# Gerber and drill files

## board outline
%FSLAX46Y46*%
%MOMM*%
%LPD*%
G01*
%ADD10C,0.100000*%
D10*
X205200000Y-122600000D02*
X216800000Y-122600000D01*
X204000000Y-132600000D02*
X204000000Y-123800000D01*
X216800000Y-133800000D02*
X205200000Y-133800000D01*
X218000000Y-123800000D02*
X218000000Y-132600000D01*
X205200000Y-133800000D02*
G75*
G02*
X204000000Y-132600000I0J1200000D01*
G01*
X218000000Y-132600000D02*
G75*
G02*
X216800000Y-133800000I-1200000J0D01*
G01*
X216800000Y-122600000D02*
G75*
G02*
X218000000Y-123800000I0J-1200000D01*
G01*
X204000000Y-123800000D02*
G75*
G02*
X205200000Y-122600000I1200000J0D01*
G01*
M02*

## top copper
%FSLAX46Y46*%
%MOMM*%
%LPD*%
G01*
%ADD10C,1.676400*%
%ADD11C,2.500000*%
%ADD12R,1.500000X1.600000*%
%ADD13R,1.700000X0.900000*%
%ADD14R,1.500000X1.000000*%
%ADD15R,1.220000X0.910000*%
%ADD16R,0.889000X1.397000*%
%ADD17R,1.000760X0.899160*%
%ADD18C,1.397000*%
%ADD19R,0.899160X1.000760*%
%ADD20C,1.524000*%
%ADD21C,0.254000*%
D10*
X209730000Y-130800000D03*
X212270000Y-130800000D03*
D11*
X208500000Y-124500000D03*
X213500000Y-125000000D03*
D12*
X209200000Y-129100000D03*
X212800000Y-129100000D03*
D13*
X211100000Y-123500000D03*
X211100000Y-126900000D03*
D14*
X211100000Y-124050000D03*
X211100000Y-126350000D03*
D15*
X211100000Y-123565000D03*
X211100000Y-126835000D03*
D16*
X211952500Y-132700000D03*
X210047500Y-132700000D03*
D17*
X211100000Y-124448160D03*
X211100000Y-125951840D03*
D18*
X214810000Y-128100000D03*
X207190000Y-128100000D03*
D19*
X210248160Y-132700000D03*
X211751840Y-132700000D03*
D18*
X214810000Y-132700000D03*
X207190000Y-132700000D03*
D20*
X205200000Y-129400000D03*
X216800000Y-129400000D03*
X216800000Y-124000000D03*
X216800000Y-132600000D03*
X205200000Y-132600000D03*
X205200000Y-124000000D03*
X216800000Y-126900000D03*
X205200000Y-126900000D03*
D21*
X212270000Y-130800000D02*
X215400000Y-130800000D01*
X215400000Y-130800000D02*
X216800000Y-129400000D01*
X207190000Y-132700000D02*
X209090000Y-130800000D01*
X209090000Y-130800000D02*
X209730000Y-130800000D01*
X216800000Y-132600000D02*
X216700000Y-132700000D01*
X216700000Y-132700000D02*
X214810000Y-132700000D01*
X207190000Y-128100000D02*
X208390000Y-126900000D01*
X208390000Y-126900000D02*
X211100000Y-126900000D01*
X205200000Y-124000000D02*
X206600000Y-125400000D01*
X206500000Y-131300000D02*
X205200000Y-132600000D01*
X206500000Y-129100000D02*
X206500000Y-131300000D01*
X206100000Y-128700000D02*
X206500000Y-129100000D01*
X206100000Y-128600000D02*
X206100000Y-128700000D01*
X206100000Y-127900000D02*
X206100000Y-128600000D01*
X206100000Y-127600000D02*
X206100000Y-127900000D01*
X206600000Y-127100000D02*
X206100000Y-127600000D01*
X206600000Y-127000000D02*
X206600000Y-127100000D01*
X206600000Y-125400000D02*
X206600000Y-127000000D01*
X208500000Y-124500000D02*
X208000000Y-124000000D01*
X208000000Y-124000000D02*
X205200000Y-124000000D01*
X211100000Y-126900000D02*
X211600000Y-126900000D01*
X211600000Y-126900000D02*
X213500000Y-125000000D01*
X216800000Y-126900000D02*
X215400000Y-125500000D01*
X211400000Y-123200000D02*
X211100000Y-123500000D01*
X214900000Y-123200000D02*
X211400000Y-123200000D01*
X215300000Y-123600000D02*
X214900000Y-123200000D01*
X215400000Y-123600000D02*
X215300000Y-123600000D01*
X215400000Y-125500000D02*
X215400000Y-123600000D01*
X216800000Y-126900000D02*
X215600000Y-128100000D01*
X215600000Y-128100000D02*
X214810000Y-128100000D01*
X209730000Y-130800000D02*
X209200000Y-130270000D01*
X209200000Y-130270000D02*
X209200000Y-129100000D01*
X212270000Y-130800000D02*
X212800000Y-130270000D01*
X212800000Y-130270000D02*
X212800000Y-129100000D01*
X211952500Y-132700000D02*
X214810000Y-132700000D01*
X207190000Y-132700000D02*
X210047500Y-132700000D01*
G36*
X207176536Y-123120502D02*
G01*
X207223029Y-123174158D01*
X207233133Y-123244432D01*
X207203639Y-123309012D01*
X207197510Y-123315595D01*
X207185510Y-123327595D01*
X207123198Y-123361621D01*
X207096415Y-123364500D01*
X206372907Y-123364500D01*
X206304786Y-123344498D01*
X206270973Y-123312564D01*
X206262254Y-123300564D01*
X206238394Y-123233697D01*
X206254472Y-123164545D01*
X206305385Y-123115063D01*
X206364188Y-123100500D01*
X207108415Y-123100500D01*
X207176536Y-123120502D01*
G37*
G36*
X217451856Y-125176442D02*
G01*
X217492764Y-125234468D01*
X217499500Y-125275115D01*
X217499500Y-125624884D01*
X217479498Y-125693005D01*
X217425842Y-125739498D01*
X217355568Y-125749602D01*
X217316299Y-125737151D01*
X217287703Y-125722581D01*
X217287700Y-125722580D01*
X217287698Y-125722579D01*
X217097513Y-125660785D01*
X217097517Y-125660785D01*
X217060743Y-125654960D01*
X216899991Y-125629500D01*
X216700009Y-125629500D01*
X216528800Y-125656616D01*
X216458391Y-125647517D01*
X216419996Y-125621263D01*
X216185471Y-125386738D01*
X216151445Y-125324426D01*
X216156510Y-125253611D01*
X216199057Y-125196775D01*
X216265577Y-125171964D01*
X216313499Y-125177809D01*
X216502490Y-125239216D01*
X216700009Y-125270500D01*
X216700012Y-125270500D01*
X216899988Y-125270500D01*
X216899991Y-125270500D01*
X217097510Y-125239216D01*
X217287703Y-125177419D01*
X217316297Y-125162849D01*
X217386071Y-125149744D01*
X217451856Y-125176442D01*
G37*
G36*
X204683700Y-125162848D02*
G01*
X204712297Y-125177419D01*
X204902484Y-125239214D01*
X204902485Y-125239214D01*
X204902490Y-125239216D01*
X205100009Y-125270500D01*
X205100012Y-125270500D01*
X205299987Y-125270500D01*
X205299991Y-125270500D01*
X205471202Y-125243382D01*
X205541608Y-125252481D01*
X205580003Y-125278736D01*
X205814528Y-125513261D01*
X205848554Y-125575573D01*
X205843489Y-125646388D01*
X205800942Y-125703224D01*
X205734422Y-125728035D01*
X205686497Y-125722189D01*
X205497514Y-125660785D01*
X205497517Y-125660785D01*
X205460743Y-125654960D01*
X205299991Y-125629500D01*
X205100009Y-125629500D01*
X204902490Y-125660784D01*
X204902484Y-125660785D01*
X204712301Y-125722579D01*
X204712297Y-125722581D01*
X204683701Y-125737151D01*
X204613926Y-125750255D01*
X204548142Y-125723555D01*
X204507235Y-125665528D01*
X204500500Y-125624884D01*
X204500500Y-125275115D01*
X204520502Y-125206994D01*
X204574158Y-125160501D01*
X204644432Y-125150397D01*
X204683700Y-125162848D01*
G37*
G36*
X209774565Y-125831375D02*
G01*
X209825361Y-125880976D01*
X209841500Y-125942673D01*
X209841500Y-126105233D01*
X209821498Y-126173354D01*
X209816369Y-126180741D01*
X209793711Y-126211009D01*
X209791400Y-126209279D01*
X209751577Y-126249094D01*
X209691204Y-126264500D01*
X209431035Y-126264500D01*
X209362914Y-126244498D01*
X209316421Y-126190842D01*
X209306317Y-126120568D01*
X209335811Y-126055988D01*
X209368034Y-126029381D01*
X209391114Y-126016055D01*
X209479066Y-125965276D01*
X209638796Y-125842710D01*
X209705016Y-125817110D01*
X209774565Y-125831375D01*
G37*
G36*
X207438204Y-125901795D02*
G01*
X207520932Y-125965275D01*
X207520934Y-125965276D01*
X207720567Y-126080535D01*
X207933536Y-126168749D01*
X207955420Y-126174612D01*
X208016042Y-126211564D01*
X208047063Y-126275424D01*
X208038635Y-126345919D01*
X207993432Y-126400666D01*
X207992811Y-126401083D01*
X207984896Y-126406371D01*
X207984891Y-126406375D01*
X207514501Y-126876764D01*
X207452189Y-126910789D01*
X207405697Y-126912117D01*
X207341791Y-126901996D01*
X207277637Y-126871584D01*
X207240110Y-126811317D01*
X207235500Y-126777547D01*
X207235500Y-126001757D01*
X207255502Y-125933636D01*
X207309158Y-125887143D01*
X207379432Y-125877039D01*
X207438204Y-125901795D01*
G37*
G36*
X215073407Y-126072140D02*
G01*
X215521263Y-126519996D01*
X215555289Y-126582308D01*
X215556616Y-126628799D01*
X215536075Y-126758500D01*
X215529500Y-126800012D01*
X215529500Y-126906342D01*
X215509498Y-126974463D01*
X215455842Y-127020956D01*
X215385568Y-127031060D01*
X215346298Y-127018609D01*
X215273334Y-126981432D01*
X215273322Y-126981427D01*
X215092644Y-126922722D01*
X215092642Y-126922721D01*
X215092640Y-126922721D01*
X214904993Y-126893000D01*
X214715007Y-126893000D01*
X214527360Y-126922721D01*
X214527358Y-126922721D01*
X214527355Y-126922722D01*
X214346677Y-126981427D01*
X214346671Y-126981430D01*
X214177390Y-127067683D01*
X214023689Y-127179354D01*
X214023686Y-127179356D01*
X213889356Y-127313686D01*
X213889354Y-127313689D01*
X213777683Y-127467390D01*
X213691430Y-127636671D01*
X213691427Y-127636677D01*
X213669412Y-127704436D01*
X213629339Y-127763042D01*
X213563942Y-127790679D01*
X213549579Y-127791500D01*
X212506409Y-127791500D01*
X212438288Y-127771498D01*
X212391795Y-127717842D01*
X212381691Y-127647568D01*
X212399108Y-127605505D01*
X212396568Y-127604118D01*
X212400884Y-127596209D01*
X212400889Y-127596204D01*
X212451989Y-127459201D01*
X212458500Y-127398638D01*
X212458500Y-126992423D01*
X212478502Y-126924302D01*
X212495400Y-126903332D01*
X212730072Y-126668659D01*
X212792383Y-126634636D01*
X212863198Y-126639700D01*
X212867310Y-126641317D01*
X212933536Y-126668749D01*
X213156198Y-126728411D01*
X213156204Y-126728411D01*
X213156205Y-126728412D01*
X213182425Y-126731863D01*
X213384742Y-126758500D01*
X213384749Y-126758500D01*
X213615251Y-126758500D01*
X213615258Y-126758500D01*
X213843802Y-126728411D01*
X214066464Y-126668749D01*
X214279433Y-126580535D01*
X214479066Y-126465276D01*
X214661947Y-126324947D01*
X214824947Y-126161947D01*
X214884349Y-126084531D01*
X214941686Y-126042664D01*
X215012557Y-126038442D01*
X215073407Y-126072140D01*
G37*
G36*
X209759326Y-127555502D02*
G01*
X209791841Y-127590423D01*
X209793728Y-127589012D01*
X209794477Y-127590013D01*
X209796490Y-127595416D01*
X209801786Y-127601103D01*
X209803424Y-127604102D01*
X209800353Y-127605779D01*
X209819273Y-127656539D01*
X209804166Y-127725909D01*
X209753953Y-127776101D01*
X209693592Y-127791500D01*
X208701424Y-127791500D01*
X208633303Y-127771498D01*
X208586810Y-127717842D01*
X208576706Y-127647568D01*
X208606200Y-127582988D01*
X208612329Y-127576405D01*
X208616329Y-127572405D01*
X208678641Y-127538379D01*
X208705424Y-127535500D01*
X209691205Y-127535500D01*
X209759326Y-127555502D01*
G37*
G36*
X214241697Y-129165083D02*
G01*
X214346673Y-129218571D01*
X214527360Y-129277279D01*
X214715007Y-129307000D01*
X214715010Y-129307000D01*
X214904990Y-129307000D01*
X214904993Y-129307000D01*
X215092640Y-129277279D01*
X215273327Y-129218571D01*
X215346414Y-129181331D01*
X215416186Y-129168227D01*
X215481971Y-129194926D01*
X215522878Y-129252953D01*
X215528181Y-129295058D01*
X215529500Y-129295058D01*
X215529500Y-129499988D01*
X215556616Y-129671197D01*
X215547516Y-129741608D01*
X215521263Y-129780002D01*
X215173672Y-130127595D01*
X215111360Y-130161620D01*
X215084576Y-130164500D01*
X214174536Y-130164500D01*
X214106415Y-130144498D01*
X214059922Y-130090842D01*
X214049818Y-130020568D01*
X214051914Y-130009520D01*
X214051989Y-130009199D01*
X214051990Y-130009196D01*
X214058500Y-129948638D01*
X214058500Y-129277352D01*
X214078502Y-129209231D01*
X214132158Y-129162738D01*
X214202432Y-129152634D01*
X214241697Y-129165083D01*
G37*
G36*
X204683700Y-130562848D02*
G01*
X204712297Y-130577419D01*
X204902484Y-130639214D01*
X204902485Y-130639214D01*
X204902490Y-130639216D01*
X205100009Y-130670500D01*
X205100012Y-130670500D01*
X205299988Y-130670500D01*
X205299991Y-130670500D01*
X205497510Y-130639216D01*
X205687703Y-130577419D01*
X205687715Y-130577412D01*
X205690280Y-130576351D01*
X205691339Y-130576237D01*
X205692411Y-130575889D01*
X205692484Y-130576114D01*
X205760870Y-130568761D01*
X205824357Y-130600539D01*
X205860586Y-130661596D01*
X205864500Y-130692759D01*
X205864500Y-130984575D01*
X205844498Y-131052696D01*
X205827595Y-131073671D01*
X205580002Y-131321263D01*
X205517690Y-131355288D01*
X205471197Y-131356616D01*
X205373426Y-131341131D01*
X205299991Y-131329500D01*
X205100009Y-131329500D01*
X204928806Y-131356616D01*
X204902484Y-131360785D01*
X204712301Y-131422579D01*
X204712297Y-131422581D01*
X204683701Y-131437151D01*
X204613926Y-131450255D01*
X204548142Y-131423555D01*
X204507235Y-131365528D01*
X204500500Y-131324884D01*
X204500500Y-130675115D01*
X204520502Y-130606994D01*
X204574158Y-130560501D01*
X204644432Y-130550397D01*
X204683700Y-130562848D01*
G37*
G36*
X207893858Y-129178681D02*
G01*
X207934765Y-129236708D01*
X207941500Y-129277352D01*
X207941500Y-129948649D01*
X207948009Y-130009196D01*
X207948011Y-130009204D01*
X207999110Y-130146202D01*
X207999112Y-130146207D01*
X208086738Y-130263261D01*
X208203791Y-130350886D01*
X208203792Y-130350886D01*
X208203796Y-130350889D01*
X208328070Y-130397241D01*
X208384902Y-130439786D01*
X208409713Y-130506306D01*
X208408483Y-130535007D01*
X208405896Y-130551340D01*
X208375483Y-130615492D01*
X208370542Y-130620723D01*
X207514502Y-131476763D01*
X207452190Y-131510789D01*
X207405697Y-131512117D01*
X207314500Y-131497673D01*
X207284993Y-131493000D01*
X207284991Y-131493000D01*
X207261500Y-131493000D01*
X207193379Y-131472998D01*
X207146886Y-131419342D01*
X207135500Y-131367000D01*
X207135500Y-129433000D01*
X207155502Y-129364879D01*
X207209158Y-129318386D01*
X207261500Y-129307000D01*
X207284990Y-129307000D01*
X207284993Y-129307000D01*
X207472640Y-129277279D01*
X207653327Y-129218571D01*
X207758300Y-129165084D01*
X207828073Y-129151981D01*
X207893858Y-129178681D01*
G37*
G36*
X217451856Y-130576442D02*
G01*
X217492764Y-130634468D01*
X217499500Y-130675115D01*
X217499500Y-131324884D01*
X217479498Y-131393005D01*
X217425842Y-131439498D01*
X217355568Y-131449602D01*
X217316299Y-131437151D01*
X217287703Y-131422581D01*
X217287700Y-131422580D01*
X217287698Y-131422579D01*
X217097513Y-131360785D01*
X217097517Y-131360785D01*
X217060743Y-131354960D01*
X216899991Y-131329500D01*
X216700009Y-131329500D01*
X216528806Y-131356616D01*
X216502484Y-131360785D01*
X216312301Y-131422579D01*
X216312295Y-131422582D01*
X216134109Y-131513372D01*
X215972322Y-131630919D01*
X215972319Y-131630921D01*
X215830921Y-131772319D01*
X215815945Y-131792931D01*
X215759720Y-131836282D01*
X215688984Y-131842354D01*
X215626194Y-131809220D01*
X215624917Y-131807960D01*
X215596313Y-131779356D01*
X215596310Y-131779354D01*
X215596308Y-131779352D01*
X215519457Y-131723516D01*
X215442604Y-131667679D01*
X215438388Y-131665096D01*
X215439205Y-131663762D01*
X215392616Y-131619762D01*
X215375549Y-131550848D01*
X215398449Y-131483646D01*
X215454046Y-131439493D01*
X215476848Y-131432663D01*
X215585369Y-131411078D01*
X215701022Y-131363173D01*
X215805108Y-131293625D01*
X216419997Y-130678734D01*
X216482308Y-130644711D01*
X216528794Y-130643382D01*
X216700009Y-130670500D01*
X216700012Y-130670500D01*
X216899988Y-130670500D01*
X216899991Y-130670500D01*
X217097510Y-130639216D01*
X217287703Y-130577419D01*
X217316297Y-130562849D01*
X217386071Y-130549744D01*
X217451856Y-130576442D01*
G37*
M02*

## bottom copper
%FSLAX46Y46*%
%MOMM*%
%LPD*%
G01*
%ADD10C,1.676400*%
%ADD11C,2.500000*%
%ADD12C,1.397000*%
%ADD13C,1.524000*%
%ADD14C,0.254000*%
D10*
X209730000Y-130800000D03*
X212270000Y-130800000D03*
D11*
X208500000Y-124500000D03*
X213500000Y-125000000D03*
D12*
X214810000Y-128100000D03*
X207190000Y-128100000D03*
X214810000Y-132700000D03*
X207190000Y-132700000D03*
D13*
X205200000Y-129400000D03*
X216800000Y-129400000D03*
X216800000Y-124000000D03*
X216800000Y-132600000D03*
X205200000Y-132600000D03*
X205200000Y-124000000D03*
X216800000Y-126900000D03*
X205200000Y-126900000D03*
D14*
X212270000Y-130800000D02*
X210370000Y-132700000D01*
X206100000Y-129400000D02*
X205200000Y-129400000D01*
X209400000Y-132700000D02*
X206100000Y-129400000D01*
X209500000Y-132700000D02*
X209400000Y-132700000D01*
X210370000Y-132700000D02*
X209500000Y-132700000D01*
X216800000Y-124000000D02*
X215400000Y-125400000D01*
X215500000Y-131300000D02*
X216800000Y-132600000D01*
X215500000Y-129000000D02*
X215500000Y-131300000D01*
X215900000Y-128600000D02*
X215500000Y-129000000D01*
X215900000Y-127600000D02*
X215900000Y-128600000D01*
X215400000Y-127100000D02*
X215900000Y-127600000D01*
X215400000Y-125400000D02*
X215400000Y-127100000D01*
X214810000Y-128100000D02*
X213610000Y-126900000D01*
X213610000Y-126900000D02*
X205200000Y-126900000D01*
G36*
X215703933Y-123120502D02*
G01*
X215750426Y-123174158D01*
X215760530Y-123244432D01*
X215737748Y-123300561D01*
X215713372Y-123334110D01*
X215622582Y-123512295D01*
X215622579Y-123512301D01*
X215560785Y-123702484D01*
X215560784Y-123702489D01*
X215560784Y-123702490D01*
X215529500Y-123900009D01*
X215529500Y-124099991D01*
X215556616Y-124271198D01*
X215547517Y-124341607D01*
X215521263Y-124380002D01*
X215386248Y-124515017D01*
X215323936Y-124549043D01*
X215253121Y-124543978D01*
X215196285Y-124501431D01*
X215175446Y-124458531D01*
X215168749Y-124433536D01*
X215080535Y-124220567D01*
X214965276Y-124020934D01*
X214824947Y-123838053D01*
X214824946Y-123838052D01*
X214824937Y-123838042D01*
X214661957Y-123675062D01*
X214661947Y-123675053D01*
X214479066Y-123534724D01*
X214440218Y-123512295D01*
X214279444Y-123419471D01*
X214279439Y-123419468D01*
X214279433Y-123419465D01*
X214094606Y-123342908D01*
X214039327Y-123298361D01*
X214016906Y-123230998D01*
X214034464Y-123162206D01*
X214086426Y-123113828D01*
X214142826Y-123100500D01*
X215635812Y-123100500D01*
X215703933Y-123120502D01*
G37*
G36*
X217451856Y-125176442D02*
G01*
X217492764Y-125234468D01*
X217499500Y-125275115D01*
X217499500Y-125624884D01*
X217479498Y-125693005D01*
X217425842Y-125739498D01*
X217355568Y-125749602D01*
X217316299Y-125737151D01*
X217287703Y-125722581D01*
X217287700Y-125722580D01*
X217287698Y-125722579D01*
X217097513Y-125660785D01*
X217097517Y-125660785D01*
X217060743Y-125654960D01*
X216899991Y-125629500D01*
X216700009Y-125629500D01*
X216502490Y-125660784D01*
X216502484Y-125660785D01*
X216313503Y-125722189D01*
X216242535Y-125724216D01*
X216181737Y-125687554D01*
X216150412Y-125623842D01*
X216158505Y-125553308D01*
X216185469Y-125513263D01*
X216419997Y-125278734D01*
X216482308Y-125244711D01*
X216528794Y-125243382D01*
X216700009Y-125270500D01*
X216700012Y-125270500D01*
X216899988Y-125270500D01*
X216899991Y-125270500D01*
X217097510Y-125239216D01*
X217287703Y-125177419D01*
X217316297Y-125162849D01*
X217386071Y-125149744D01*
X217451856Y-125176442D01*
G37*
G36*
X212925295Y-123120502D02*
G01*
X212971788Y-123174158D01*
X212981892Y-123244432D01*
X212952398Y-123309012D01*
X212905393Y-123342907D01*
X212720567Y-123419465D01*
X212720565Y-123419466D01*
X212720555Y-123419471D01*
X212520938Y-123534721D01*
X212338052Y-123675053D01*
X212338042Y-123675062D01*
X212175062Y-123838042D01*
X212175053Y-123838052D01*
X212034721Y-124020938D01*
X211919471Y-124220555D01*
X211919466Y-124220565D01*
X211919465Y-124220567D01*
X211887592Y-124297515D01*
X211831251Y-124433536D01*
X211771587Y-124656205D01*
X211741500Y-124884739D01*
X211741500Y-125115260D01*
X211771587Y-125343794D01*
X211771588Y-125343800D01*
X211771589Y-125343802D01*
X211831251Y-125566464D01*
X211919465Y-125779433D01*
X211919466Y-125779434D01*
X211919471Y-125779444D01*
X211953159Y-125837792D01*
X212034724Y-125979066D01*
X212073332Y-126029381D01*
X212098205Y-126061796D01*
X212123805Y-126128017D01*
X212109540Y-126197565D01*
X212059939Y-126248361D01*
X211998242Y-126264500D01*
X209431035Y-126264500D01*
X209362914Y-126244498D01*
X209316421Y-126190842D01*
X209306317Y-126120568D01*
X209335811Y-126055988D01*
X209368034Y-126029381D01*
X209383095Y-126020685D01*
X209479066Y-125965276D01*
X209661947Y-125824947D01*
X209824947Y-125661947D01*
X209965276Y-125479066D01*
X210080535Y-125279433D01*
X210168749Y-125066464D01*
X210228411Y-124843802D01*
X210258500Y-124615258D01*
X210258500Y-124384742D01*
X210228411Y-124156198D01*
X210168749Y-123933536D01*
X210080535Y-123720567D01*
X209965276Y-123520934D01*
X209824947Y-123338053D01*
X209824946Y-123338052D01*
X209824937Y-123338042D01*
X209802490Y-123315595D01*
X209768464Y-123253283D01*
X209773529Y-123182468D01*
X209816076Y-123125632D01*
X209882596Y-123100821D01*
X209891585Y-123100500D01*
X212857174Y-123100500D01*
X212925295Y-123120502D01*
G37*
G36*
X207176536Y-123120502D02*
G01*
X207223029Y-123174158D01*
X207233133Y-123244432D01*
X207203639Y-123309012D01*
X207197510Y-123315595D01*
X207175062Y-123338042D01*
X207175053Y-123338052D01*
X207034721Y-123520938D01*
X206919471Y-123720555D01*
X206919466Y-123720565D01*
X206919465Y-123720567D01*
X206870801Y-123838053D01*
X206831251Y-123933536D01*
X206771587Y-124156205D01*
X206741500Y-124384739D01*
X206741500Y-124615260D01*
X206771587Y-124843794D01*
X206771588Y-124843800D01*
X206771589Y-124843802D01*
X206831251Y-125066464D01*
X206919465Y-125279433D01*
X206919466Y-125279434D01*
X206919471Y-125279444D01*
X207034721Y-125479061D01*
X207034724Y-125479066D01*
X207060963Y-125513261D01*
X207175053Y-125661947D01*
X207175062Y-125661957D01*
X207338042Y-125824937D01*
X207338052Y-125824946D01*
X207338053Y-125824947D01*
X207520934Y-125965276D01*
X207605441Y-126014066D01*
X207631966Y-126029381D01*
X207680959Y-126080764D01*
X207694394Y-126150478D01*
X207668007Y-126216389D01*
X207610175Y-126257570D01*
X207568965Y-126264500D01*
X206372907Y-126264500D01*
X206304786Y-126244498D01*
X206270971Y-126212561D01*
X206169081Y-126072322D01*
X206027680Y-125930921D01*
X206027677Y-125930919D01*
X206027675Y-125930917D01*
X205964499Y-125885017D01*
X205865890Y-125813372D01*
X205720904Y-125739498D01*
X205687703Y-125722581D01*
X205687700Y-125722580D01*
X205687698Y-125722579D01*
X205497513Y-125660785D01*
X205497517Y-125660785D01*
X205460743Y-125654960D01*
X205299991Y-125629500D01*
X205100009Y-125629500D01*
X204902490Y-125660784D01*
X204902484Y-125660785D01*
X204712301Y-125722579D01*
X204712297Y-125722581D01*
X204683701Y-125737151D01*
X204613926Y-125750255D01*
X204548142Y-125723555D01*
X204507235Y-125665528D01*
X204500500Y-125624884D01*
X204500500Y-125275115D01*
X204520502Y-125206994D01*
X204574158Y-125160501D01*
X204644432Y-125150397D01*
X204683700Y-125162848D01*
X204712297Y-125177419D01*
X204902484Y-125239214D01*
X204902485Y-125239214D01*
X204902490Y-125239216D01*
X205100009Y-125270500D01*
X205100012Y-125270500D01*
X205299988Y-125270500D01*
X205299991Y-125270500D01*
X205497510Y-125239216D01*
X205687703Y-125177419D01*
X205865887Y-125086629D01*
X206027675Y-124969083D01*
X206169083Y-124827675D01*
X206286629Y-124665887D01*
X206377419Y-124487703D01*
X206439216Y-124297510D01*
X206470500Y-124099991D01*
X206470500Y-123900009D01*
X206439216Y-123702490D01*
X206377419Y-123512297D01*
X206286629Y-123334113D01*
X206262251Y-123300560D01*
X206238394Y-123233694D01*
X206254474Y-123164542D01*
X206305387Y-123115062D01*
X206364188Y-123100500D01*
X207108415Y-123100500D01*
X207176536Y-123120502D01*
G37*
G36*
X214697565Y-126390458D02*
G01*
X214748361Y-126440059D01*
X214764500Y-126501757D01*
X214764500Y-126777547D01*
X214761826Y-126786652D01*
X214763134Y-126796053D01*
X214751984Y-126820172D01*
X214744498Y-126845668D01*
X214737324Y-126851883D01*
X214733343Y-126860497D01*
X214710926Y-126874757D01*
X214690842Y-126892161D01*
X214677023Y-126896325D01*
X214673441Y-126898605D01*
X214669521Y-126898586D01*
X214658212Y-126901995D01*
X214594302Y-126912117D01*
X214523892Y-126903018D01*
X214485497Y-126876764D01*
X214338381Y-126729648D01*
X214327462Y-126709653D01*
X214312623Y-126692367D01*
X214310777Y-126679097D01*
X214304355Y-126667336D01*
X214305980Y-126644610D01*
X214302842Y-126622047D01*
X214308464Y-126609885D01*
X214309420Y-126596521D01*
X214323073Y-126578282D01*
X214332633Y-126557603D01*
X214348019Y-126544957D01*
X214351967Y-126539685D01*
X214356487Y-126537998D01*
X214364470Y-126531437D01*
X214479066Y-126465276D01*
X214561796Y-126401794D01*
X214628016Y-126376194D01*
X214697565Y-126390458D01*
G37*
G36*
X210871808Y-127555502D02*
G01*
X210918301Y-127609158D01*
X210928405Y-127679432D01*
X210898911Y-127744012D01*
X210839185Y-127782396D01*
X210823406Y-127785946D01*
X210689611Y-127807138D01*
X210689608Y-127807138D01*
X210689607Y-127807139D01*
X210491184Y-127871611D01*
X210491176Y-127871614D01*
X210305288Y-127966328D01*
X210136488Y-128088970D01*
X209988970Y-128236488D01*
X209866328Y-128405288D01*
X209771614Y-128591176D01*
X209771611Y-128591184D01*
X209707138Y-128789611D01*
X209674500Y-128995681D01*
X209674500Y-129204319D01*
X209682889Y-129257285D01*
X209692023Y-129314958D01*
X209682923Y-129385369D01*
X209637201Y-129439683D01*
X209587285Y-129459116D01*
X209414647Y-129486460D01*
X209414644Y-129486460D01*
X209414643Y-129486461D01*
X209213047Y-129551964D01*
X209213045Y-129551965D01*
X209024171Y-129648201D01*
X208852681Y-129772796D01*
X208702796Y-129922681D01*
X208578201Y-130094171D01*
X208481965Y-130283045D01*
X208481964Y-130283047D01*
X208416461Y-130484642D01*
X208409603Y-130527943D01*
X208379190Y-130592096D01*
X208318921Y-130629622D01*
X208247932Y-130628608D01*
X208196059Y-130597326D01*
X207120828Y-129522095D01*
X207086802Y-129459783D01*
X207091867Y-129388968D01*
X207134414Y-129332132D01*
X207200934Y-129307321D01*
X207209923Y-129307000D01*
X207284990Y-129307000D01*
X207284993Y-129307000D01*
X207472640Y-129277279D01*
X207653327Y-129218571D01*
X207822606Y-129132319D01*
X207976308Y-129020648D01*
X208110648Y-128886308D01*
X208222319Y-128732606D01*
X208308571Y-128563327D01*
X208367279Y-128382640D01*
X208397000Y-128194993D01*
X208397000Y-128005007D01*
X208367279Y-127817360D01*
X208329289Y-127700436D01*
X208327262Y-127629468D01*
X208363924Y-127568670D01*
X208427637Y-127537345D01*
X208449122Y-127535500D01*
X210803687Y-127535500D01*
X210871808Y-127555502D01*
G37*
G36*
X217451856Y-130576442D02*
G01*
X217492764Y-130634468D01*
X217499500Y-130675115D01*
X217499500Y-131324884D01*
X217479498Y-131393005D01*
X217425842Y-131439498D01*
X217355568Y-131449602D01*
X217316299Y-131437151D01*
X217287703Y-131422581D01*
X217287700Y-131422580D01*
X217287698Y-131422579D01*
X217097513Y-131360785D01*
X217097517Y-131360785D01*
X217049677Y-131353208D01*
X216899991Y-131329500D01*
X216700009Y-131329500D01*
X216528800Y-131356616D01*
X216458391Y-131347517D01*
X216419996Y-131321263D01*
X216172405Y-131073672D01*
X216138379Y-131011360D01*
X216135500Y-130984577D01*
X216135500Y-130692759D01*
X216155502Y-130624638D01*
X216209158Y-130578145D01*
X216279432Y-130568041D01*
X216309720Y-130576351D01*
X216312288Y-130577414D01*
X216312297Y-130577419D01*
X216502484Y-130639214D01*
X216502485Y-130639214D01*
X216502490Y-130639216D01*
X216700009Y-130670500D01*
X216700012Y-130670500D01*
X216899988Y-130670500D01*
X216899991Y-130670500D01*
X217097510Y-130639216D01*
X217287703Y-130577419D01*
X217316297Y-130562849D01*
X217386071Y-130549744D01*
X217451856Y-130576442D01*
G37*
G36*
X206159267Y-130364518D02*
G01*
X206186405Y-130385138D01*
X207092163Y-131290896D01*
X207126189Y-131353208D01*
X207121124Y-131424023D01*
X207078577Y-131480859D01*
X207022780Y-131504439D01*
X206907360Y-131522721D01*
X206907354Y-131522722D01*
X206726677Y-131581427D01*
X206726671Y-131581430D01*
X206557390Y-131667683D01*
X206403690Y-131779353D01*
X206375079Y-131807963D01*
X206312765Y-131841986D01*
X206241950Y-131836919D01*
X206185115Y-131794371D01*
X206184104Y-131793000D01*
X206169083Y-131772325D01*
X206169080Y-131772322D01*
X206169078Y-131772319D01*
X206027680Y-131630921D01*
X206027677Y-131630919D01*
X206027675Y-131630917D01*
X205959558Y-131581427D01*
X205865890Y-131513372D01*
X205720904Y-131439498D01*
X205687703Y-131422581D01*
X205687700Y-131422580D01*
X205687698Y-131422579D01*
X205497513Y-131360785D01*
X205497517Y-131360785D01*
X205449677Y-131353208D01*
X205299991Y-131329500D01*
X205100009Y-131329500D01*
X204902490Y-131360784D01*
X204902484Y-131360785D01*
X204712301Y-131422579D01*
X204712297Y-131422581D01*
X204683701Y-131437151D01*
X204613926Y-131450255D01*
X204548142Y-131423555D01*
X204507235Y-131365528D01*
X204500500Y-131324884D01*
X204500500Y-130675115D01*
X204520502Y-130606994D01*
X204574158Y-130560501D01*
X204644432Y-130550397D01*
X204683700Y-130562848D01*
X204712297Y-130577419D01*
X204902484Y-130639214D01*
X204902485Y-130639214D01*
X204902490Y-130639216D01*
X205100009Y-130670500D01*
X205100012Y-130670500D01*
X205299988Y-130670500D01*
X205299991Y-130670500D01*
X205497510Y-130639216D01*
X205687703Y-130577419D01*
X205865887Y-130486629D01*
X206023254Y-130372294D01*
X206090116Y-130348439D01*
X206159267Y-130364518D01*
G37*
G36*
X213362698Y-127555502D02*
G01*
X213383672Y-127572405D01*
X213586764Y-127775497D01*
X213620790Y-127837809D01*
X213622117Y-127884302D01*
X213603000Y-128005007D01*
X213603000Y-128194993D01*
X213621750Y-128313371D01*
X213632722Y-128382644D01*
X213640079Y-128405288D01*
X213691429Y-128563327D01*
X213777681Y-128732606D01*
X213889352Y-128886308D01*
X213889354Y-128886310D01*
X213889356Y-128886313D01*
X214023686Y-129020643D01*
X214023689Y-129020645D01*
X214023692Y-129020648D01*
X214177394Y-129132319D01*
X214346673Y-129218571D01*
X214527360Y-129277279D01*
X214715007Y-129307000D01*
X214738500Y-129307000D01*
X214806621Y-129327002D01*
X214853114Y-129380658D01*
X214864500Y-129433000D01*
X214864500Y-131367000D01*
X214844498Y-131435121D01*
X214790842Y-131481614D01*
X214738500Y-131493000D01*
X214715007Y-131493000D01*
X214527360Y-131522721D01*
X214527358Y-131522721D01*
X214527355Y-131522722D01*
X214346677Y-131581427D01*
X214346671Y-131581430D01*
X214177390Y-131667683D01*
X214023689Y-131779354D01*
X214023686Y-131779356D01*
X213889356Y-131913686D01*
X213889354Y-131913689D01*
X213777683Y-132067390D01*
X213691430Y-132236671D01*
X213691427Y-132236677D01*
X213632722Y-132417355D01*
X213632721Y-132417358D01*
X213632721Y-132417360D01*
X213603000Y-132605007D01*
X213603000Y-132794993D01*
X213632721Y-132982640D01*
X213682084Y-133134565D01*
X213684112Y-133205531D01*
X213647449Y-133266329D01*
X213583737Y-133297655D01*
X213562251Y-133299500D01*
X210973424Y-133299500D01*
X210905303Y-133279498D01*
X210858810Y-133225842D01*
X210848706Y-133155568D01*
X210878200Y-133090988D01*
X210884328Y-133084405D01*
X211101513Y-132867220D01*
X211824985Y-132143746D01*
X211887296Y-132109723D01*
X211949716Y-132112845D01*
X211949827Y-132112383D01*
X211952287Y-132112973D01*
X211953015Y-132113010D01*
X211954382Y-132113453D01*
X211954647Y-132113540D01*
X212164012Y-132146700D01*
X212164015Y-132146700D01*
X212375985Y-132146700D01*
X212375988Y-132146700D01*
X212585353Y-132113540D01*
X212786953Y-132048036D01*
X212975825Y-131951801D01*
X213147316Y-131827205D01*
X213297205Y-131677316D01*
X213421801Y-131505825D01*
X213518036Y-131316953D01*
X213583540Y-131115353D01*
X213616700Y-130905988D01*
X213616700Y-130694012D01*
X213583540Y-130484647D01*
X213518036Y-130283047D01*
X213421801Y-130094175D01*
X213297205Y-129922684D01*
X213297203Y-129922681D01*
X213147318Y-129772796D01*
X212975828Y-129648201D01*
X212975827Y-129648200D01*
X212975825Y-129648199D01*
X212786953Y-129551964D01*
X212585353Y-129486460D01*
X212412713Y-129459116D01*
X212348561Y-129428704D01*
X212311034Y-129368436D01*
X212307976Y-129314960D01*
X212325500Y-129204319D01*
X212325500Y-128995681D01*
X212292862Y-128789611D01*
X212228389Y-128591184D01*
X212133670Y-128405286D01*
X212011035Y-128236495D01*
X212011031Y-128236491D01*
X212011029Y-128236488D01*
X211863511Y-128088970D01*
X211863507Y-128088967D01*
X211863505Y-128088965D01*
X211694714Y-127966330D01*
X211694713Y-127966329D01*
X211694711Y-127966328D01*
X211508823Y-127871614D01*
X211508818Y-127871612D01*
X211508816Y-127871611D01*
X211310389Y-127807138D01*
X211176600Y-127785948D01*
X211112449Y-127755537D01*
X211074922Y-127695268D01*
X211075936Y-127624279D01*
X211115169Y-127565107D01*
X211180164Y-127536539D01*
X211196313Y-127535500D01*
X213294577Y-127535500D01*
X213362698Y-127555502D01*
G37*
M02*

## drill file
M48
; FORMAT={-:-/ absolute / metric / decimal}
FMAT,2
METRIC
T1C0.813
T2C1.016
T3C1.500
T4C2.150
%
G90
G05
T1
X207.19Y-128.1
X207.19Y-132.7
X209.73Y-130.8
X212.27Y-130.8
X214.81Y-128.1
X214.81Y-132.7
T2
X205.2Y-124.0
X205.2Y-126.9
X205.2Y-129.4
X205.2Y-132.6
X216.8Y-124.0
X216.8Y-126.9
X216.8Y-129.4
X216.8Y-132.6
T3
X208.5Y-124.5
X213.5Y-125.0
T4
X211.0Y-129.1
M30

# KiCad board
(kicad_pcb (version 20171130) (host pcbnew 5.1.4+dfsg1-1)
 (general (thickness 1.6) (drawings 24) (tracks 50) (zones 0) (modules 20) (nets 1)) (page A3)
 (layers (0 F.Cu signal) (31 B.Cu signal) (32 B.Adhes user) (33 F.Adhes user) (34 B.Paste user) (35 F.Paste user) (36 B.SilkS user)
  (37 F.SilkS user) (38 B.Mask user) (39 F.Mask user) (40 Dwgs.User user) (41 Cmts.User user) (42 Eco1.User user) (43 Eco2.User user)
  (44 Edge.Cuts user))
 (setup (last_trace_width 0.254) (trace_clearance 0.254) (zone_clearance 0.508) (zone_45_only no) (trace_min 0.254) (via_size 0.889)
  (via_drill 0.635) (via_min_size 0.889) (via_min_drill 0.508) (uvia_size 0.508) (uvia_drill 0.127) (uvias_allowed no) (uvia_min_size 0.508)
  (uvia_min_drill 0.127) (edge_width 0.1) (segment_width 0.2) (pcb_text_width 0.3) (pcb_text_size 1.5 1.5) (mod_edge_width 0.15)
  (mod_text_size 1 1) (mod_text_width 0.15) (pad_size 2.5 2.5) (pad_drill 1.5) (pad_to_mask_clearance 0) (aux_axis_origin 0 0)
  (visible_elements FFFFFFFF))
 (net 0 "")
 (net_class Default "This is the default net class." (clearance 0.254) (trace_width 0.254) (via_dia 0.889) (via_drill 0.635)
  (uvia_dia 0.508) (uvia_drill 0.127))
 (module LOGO (layer B.Cu) (at 211.1 124)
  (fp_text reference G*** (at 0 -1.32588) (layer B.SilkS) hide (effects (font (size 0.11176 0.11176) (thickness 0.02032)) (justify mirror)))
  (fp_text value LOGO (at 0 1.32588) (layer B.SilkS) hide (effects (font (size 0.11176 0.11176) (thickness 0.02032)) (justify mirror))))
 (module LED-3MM (layer F.Cu) (at 211 130.8)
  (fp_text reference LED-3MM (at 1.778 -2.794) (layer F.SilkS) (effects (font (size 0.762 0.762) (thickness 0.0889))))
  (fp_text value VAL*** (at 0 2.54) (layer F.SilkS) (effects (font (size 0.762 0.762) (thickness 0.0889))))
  (pad 1 thru_hole circle (at -1.27 0) (size 1.6764 1.6764) (drill 0.8128) (layers *.Cu *.Mask F.SilkS))
  (pad 2 thru_hole circle (at 1.27 0) (size 1.6764 1.6764) (drill 0.8128) (layers *.Cu *.Mask F.SilkS)))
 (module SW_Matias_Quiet (layer F.Cu) (at 211 129)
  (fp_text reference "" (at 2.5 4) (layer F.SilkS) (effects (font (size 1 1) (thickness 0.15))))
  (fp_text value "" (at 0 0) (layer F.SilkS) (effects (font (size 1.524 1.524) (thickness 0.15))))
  (pad 1 thru_hole circle (at -2.5 -4.5) (size 2.5 2.5) (drill 1.5) (layers *.Cu *.Mask F.SilkS))
  (pad 2 thru_hole circle (at 2.5 -4) (size 2.5 2.5) (drill 1.5) (layers *.Cu *.Mask F.SilkS)))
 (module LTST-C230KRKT (layer F.Cu) (at 211 129.1)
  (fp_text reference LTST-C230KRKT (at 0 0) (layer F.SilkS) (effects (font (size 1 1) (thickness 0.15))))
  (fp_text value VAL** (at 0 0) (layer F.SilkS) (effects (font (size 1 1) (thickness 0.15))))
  (pad 2 smd rect (at -1.8 0) (size 1.5 1.6) (layers F.Cu F.Paste F.Mask))
  (pad 3 smd rect (at 1.8 0) (size 1.5 1.6) (layers F.Cu F.Paste F.Mask))
  (pad "" np_thru_hole circle (at 0 0) (size 2.15 2.15) (drill 2.15) (layers *.Cu *.Mask F.SilkS)))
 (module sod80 (layer F.Cu) (at 211.1 125.2 90)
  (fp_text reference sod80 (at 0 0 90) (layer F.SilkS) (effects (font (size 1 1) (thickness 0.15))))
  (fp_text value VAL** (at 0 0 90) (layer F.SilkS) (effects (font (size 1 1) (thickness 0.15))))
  (pad 5 smd rect (at 1.7 0 90) (size 0.9 1.7) (layers F.Cu F.Paste F.Mask))
  (pad 6 smd rect (at -1.7 0 90) (size 0.9 1.7) (layers F.Cu F.Paste F.Mask)))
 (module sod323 (layer F.Cu) (at 211.1 125.2 90)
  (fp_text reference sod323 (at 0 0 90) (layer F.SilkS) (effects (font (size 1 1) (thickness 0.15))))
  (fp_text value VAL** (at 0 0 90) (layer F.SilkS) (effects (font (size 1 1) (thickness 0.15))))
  (pad 3 smd rect (at 1.15 0 90) (size 1 1.5) (layers F.Cu F.Paste F.Mask))
  (pad 4 smd rect (at -1.15 0 90) (size 1 1.5) (layers F.Cu F.Paste F.Mask)))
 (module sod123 (layer F.Cu) (at 211.1 125.2 90)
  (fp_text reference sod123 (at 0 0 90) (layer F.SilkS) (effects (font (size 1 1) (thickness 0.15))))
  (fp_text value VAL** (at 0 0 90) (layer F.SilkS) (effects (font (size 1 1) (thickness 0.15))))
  (pad 1 smd rect (at 1.635 0 90) (size 0.91 1.22) (layers F.Cu F.Paste F.Mask))
  (pad 2 smd rect (at -1.635 0 90) (size 0.91 1.22) (layers F.Cu F.Paste F.Mask)))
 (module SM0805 (layer F.Cu) (at 211 132.7 180)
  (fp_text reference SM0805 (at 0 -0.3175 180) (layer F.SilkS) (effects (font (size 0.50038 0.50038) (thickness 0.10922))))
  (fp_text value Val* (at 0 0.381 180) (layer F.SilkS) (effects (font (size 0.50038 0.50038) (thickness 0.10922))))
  (pad 1 smd rect (at -0.9525 0 180) (size 0.889 1.397) (layers F.Cu F.Paste F.Mask))
  (pad 2 smd rect (at 0.9525 0 180) (size 0.889 1.397) (layers F.Cu F.Paste F.Mask)))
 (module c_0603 (layer F.Cu) (at 211.1 125.2 90)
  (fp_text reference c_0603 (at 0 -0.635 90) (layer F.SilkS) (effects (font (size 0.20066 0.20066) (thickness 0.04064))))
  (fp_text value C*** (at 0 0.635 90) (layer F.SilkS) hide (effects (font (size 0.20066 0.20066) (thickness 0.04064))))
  (pad 1 smd rect (at 0.75184 0 90) (size 0.89916 1.00076) (layers F.Cu F.Paste F.Mask))
  (pad 2 smd rect (at -0.75184 0 90) (size 0.89916 1.00076) (layers F.Cu F.Paste F.Mask)))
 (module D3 (layer F.Cu) (at 211 128.1)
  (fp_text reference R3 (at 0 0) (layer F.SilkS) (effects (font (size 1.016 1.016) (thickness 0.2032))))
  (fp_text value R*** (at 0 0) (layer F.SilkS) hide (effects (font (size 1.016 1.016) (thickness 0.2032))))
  (pad 2 thru_hole circle (at 3.81 0) (size 1.397 1.397) (drill 0.8128) (layers *.Cu *.Mask F.SilkS))
  (pad 1 thru_hole circle (at -3.81 0) (size 1.397 1.397) (drill 0.8128) (layers *.Cu *.Mask F.SilkS)))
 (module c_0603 (layer F.Cu) (at 211 132.7 180)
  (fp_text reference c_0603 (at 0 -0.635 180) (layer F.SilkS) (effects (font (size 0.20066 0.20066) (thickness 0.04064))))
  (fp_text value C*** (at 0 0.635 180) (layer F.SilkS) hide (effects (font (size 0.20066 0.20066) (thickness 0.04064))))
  (pad 1 smd rect (at 0.75184 0 180) (size 0.89916 1.00076) (layers F.Cu F.Paste F.Mask))
  (pad 2 smd rect (at -0.75184 0 180) (size 0.89916 1.00076) (layers F.Cu F.Paste F.Mask)))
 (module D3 (layer F.Cu) (at 211 132.7)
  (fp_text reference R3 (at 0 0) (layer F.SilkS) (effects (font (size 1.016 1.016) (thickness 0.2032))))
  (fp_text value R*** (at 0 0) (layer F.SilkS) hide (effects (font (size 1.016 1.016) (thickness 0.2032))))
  (pad 2 thru_hole circle (at 3.81 0) (size 1.397 1.397) (drill 0.8128) (layers *.Cu *.Mask F.SilkS))
  (pad 1 thru_hole circle (at -3.81 0) (size 1.397 1.397) (drill 0.8128) (layers *.Cu *.Mask F.SilkS)))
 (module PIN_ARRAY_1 (layer F.Cu) (at 205.2 129.4)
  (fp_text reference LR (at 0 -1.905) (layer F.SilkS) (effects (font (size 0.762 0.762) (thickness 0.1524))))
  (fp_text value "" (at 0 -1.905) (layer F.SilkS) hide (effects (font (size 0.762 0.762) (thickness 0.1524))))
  (pad 1 thru_hole circle (at 0 0) (size 1.524 1.524) (drill 1.016) (layers *.Cu *.Mask F.SilkS)))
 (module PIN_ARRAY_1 (layer F.Cu) (at 216.8 129.4)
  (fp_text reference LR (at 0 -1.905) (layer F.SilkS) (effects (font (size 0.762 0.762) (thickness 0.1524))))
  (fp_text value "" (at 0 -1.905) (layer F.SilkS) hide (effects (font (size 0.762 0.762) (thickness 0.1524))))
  (pad 1 thru_hole circle (at 0 0) (size 1.524 1.524) (drill 1.016) (layers *.Cu *.Mask F.SilkS)))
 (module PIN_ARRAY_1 (layer F.Cu) (at 216.8 124)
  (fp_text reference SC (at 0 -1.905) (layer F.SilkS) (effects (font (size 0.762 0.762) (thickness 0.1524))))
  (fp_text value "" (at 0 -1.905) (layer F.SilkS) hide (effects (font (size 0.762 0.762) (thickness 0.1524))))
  (pad 1 thru_hole circle (at 0 0) (size 1.524 1.524) (drill 1.016) (layers *.Cu *.Mask F.SilkS)))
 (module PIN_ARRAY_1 (layer F.Cu) (at 216.8 132.6)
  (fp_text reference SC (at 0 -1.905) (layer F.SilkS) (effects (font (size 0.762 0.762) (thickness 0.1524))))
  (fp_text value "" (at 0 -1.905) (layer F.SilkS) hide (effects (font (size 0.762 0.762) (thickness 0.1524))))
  (pad 1 thru_hole circle (at 0 0) (size 1.524 1.524) (drill 1.016) (layers *.Cu *.Mask F.SilkS)))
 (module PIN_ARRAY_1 (layer F.Cu) (at 205.2 132.6)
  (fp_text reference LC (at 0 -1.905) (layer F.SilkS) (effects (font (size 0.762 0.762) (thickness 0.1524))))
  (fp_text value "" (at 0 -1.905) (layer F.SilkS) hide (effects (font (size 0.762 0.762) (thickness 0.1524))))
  (pad 1 thru_hole circle (at 0 0) (size 1.524 1.524) (drill 1.016) (layers *.Cu *.Mask F.SilkS)))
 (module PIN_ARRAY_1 (layer F.Cu) (at 205.2 124)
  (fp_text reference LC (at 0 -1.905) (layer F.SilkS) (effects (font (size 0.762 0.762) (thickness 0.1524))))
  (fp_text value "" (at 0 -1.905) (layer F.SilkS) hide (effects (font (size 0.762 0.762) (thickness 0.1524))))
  (pad 1 thru_hole circle (at 0 0) (size 1.524 1.524) (drill 1.016) (layers *.Cu *.Mask F.SilkS)))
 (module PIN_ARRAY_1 (layer F.Cu) (at 216.8 126.9)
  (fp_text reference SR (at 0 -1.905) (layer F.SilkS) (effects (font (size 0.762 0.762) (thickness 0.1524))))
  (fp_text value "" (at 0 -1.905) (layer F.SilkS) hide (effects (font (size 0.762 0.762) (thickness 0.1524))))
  (pad 1 thru_hole circle (at 0 0) (size 1.524 1.524) (drill 1.016) (layers *.Cu *.Mask F.SilkS)))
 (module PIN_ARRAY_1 (layer F.Cu) (at 205.2 126.9)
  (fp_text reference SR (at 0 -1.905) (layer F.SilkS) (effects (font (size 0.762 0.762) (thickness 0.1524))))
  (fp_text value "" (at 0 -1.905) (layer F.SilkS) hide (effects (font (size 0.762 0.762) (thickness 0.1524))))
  (pad 1 thru_hole circle (at 0 0) (size 1.524 1.524) (drill 1.016) (layers *.Cu *.Mask F.SilkS)))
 (gr_line (start 205.2 122.6) (end 216.8 122.6) (angle 90) (layer Edge.Cuts) (width 0.1))
 (gr_line (start 204 132.6) (end 204 123.8) (angle 90) (layer Edge.Cuts) (width 0.1))
 (gr_line (start 216.8 133.8) (end 205.2 133.8) (angle 90) (layer Edge.Cuts) (width 0.1))
 (gr_line (start 218 123.8) (end 218 132.6) (angle 90) (layer Edge.Cuts) (width 0.1))
 (gr_arc (start 205.2 132.6) (end 205.2 133.8) (angle 90) (layer Edge.Cuts) (width 0.1))
 (gr_arc (start 216.8 132.6) (end 218 132.6) (angle 90) (layer Edge.Cuts) (width 0.1))
 (gr_arc (start 216.8 123.8) (end 216.8 122.6) (angle 90) (layer Edge.Cuts) (width 0.1))
 (gr_arc (start 205.2 123.8) (end 204 123.8) (angle 90) (layer Edge.Cuts) (width 0.1))
 (segment (start 212.27 130.8) (end 215.4 130.8) (width 0.254) (layer F.Cu) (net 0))
 (segment (start 215.4 130.8) (end 216.8 129.4) (width 0.254) (layer F.Cu) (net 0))
 (segment (start 212.27 130.8) (end 210.37 132.7) (width 0.254) (layer B.Cu) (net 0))
 (segment (start 206.1 129.4) (end 205.2 129.4) (width 0.254) (layer B.Cu) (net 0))
 (segment (start 209.4 132.7) (end 206.1 129.4) (width 0.254) (layer B.Cu) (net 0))
 (segment (start 209.5 132.7) (end 209.4 132.7) (width 0.254) (layer B.Cu) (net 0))
 (segment (start 210.37 132.7) (end 209.5 132.7) (width 0.254) (layer B.Cu) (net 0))
 (segment (start 207.19 132.7) (end 209.09 130.8) (width 0.254) (layer F.Cu) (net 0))
 (segment (start 209.09 130.8) (end 209.73 130.8) (width 0.254) (layer F.Cu) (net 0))
 (segment (start 216.8 132.6) (end 216.7 132.7) (width 0.254) (layer F.Cu) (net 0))
 (segment (start 216.7 132.7) (end 214.81 132.7) (width 0.254) (layer F.Cu) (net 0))
 (segment (start 216.8 124) (end 215.4 125.4) (width 0.254) (layer B.Cu) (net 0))
 (segment (start 215.5 131.3) (end 216.8 132.6) (width 0.254) (layer B.Cu) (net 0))
 (segment (start 215.5 129) (end 215.5 131.3) (width 0.254) (layer B.Cu) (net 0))
 (segment (start 215.9 128.6) (end 215.5 129) (width 0.254) (layer B.Cu) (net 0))
 (segment (start 215.9 127.6) (end 215.9 128.6) (width 0.254) (layer B.Cu) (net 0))
 (segment (start 215.4 127.1) (end 215.9 127.6) (width 0.254) (layer B.Cu) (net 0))
 (segment (start 215.4 125.4) (end 215.4 127.1) (width 0.254) (layer B.Cu) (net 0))
 (segment (start 207.19 128.1) (end 208.39 126.9) (width 0.254) (layer F.Cu) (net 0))
 (segment (start 208.39 126.9) (end 211.1 126.9) (width 0.254) (layer F.Cu) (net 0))
 (segment (start 205.2 124) (end 206.6 125.4) (width 0.254) (layer F.Cu) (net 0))
 (segment (start 206.5 131.3) (end 205.2 132.6) (width 0.254) (layer F.Cu) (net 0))
 (segment (start 206.5 129.1) (end 206.5 131.3) (width 0.254) (layer F.Cu) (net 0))
 (segment (start 206.1 128.7) (end 206.5 129.1) (width 0.254) (layer F.Cu) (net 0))
 (segment (start 206.1 128.6) (end 206.1 128.7) (width 0.254) (layer F.Cu) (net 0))
 (segment (start 206.1 127.9) (end 206.1 128.6) (width 0.254) (layer F.Cu) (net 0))
 (segment (start 206.1 127.6) (end 206.1 127.9) (width 0.254) (layer F.Cu) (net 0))
 (segment (start 206.6 127.1) (end 206.1 127.6) (width 0.254) (layer F.Cu) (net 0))
 (segment (start 206.6 127) (end 206.6 127.1) (width 0.254) (layer F.Cu) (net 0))
 (segment (start 206.6 125.4) (end 206.6 127) (width 0.254) (layer F.Cu) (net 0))
 (segment (start 214.81 128.1) (end 213.61 126.9) (width 0.254) (layer B.Cu) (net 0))
 (segment (start 213.61 126.9) (end 205.2 126.9) (width 0.254) (layer B.Cu) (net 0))
 (segment (start 208.5 124.5) (end 208 124) (width 0.254) (layer F.Cu) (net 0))
 (segment (start 208 124) (end 205.2 124) (width 0.254) (layer F.Cu) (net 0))
 (segment (start 211.1 126.9) (end 211.6 126.9) (width 0.254) (layer F.Cu) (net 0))
 (segment (start 211.6 126.9) (end 213.5 125) (width 0.254) (layer F.Cu) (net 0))
 (segment (start 216.8 126.9) (end 215.4 125.5) (width 0.254) (layer F.Cu) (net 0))
 (segment (start 211.4 123.2) (end 211.1 123.5) (width 0.254) (layer F.Cu) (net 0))
 (segment (start 214.9 123.2) (end 211.4 123.2) (width 0.254) (layer F.Cu) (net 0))
 (segment (start 215.3 123.6) (end 214.9 123.2) (width 0.254) (layer F.Cu) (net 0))
 (segment (start 215.4 123.6) (end 215.3 123.6) (width 0.254) (layer F.Cu) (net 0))
 (segment (start 215.4 125.5) (end 215.4 123.6) (width 0.254) (layer F.Cu) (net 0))
 (segment (start 216.8 126.9) (end 215.6 128.1) (width 0.254) (layer F.Cu) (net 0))
 (segment (start 215.6 128.1) (end 214.81 128.1) (width 0.254) (layer F.Cu) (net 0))
 (segment (start 209.73 130.8) (end 209.2 130.27) (width 0.254) (layer F.Cu) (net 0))
 (segment (start 209.2 130.27) (end 209.2 129.1) (width 0.254) (layer F.Cu) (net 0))
 (segment (start 212.27 130.8) (end 212.8 130.27) (width 0.254) (layer F.Cu) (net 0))
 (segment (start 212.8 130.27) (end 212.8 129.1) (width 0.254) (layer F.Cu) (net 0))
 (segment (start 211.9525 132.7) (end 214.81 132.7) (width 0.254) (layer F.Cu) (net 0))
 (segment (start 207.19 132.7) (end 210.0475 132.7) (width 0.254) (layer F.Cu) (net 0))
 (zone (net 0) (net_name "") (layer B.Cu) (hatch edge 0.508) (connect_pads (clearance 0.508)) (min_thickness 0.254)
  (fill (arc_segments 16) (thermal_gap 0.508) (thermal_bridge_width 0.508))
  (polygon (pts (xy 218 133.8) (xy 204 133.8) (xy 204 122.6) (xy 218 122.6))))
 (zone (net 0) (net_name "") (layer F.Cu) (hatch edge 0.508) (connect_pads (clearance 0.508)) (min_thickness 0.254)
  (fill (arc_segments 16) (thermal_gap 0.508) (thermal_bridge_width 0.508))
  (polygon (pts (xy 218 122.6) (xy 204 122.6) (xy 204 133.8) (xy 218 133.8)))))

